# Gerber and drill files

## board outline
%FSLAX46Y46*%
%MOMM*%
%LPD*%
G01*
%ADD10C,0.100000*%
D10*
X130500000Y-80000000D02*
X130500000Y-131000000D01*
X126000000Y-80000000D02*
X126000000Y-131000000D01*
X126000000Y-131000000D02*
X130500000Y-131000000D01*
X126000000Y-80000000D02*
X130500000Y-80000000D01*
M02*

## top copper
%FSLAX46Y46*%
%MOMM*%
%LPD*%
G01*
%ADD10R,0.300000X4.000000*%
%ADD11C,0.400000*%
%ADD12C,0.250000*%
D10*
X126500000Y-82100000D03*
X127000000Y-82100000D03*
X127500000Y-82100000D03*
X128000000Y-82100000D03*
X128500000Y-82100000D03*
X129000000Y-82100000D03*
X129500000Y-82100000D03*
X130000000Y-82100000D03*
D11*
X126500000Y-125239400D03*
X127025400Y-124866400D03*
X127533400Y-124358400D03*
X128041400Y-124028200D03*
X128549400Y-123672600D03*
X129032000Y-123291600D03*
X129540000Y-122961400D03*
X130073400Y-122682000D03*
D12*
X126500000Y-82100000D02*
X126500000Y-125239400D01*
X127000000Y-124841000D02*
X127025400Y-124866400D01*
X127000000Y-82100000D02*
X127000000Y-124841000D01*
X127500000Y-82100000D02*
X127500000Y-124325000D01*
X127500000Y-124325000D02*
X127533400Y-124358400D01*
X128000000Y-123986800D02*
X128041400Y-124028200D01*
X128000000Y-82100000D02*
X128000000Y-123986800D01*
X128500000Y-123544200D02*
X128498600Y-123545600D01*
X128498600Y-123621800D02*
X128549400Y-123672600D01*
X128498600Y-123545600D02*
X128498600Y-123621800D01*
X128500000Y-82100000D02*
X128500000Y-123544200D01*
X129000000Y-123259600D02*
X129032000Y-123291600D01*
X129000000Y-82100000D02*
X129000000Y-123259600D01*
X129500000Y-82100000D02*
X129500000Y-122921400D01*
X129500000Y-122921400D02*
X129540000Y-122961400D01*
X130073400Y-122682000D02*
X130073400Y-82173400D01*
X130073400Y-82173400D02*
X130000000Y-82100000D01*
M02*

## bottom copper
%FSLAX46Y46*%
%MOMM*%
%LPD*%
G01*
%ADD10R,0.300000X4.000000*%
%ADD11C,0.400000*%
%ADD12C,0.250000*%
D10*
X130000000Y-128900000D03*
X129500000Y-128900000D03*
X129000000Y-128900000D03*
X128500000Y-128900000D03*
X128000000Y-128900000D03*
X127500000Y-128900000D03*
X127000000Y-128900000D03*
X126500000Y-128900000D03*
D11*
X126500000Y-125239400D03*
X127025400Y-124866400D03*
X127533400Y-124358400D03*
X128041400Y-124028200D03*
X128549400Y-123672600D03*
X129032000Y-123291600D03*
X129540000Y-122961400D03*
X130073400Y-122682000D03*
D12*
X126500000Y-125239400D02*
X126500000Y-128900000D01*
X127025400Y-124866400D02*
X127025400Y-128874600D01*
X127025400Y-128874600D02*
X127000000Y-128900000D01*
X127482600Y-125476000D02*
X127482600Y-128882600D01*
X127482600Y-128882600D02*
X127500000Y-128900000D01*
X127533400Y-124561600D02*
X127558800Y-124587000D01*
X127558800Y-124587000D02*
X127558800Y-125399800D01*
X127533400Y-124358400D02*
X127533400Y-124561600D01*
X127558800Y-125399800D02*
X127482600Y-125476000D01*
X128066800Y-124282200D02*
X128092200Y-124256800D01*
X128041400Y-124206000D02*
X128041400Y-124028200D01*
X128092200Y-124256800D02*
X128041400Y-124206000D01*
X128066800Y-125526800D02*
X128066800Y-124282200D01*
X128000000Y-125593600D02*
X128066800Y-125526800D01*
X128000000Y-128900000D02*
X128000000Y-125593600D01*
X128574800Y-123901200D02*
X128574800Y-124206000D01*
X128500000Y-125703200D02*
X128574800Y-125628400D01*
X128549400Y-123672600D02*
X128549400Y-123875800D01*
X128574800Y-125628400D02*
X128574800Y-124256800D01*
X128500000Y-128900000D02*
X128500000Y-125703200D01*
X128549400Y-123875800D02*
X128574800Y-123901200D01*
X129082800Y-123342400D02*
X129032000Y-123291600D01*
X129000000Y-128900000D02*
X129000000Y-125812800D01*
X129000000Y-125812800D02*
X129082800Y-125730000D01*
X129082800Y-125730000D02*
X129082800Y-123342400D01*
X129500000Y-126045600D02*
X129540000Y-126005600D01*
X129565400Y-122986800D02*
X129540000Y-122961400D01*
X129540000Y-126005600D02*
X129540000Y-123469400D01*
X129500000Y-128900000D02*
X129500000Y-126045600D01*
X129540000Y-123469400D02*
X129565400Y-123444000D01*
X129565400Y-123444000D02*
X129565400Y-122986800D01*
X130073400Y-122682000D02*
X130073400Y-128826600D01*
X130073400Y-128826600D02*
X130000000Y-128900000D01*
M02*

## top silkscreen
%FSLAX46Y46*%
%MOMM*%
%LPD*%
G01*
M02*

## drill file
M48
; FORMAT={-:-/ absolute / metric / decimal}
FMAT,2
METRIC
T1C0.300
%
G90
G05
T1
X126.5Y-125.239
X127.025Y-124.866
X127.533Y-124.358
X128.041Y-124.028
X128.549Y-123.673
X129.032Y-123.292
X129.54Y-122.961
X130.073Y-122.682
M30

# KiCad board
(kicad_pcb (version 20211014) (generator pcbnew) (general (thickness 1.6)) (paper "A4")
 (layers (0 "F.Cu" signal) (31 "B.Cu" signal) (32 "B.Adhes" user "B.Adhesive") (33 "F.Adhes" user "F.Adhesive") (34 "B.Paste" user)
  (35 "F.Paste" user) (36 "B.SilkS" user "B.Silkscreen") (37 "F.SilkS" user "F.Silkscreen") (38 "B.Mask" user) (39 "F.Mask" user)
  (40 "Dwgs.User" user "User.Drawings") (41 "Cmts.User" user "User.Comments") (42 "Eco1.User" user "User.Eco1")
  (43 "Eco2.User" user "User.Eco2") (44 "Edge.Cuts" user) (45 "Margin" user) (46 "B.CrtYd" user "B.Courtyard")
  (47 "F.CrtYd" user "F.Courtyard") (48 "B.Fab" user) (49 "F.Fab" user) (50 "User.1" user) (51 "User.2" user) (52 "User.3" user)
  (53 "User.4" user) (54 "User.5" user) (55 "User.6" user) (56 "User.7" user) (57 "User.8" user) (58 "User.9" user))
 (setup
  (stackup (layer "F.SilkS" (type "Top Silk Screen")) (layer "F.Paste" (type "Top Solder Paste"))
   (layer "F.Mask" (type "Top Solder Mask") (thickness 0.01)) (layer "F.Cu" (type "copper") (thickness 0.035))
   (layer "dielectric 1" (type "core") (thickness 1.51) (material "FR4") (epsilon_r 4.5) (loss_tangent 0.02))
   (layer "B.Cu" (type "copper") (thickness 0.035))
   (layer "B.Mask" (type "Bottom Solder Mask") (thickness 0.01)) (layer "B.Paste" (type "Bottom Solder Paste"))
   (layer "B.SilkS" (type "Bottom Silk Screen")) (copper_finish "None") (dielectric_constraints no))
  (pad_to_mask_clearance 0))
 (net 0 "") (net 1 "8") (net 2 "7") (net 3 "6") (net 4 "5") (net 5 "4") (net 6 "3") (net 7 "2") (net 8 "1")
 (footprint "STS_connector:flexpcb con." (layer "F.Cu") (at 126 84.1)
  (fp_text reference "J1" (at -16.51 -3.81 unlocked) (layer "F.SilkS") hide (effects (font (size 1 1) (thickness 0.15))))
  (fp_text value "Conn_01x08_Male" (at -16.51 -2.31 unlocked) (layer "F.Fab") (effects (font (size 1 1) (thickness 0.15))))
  (pad "1" smd rect (at 0.5 -2) (size 0.3 4) (layers "F.Cu" "F.Paste" "F.Mask") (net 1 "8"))
  (pad "2" smd rect (at 1 -2) (size 0.3 4) (layers "F.Cu" "F.Paste" "F.Mask") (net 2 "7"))
  (pad "3" smd rect (at 1.5 -2) (size 0.3 4) (layers "F.Cu" "F.Paste" "F.Mask") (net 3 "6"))
  (pad "4" smd rect (at 2 -2) (size 0.3 4) (layers "F.Cu" "F.Paste" "F.Mask") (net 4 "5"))
  (pad "5" smd rect (at 2.5 -2) (size 0.3 4) (layers "F.Cu" "F.Paste" "F.Mask") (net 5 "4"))
  (pad "6" smd rect (at 3 -2) (size 0.3 4) (layers "F.Cu" "F.Paste" "F.Mask") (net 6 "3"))
  (pad "7" smd rect (at 3.5 -2) (size 0.3 4) (layers "F.Cu" "F.Paste" "F.Mask") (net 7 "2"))
  (pad "8" smd rect (at 4 -2) (size 0.3 4) (layers "F.Cu" "F.Paste" "F.Mask") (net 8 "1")))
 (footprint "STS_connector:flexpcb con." (layer "B.Cu") (at 130.5 130.9 180)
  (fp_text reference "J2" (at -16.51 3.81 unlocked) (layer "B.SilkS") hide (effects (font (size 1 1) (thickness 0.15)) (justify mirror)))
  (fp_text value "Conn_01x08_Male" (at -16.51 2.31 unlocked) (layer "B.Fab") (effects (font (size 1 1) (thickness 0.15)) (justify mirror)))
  (pad "1" smd rect (at 0.5 2 180) (size 0.3 4) (layers "B.Cu" "B.Paste" "B.Mask") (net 8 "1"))
  (pad "2" smd rect (at 1 2 180) (size 0.3 4) (layers "B.Cu" "B.Paste" "B.Mask") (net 7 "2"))
  (pad "3" smd rect (at 1.5 2 180) (size 0.3 4) (layers "B.Cu" "B.Paste" "B.Mask") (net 6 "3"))
  (pad "4" smd rect (at 2 2 180) (size 0.3 4) (layers "B.Cu" "B.Paste" "B.Mask") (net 5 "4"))
  (pad "5" smd rect (at 2.5 2 180) (size 0.3 4) (layers "B.Cu" "B.Paste" "B.Mask") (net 4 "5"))
  (pad "6" smd rect (at 3 2 180) (size 0.3 4) (layers "B.Cu" "B.Paste" "B.Mask") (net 3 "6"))
  (pad "7" smd rect (at 3.5 2 180) (size 0.3 4) (layers "B.Cu" "B.Paste" "B.Mask") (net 2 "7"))
  (pad "8" smd rect (at 4 2 180) (size 0.3 4) (layers "B.Cu" "B.Paste" "B.Mask") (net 1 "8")))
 (gr_line (start 130.5 80) (end 130.5 131) (layer "Edge.Cuts") (width 0.1))
 (gr_line (start 126 80) (end 126 131) (layer "Edge.Cuts") (width 0.1))
 (gr_line (start 126 131) (end 130.5 131) (layer "Edge.Cuts") (width 0.1))
 (gr_line (start 126 80) (end 130.5 80) (layer "Edge.Cuts") (width 0.1))
 (segment (start 126.5 82.1) (end 126.5 125.2394) (width 0.25) (layer "F.Cu") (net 1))
 (via (at 126.5 125.2394) (size 0.4) (drill 0.3) (layers "F.Cu" "B.Cu") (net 1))
 (segment (start 126.5 125.2394) (end 126.5 128.9) (width 0.25) (layer "B.Cu") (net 1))
 (segment (start 127 124.841) (end 127.0254 124.8664) (width 0.25) (layer "F.Cu") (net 2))
 (segment (start 127 82.1) (end 127 124.841) (width 0.25) (layer "F.Cu") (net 2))
 (via (at 127.0254 124.8664) (size 0.4) (drill 0.3) (layers "F.Cu" "B.Cu") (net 2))
 (segment (start 127.0254 124.8664) (end 127.0254 128.8746) (width 0.25) (layer "B.Cu") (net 2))
 (segment (start 127.0254 128.8746) (end 127 128.9) (width 0.25) (layer "B.Cu") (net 2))
 (segment (start 127.5 82.1) (end 127.5 124.325) (width 0.25) (layer "F.Cu") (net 3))
 (segment (start 127.5 124.325) (end 127.5334 124.3584) (width 0.25) (layer "F.Cu") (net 3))
 (via (at 127.5334 124.3584) (size 0.4) (drill 0.3) (layers "F.Cu" "B.Cu") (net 3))
 (segment (start 127.4826 125.476) (end 127.4826 128.8826) (width 0.25) (layer "B.Cu") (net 3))
 (segment (start 127.4826 128.8826) (end 127.5 128.9) (width 0.25) (layer "B.Cu") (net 3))
 (segment (start 127.5334 124.5616) (end 127.5588 124.587) (width 0.25) (layer "B.Cu") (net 3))
 (segment (start 127.5588 124.587) (end 127.5588 125.3998) (width 0.25) (layer "B.Cu") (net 3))
 (segment (start 127.5334 124.3584) (end 127.5334 124.5616) (width 0.25) (layer "B.Cu") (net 3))
 (segment (start 127.5588 125.3998) (end 127.4826 125.476) (width 0.25) (layer "B.Cu") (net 3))
 (segment (start 128 123.9868) (end 128.0414 124.0282) (width 0.25) (layer "F.Cu") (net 4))
 (segment (start 128 82.1) (end 128 123.9868) (width 0.25) (layer "F.Cu") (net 4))
 (via (at 128.0414 124.0282) (size 0.4) (drill 0.3) (layers "F.Cu" "B.Cu") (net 4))
 (segment (start 128.0668 124.2822) (end 128.0922 124.2568) (width 0.25) (layer "B.Cu") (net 4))
 (segment (start 128.0414 124.206) (end 128.0414 124.0282) (width 0.25) (layer "B.Cu") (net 4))
 (segment (start 128.0922 124.2568) (end 128.0414 124.206) (width 0.25) (layer "B.Cu") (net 4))
 (segment (start 128.0668 125.5268) (end 128.0668 124.2822) (width 0.25) (layer "B.Cu") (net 4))
 (segment (start 128 125.5936) (end 128.0668 125.5268) (width 0.25) (layer "B.Cu") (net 4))
 (segment (start 128 128.9) (end 128 125.5936) (width 0.25) (layer "B.Cu") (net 4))
 (segment (start 128.5 123.5442) (end 128.4986 123.5456) (width 0.25) (layer "F.Cu") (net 5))
 (segment (start 128.4986 123.6218) (end 128.5494 123.6726) (width 0.25) (layer "F.Cu") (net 5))
 (segment (start 128.4986 123.5456) (end 128.4986 123.6218) (width 0.25) (layer "F.Cu") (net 5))
 (segment (start 128.5 82.1) (end 128.5 123.5442) (width 0.25) (layer "F.Cu") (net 5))
 (via (at 128.5494 123.6726) (size 0.4) (drill 0.3) (layers "F.Cu" "B.Cu") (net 5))
 (segment (start 128.5748 123.9012) (end 128.5748 124.206) (width 0.25) (layer "B.Cu") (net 5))
 (segment (start 128.5 125.7032) (end 128.5748 125.6284) (width 0.25) (layer "B.Cu") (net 5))
 (segment (start 128.5494 123.6726) (end 128.5494 123.8758) (width 0.25) (layer "B.Cu") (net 5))
 (segment (start 128.5748 125.6284) (end 128.5748 124.2568) (width 0.25) (layer "B.Cu") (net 5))
 (segment (start 128.5 128.9) (end 128.5 125.7032) (width 0.25) (layer "B.Cu") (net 5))
 (segment (start 128.5494 123.8758) (end 128.5748 123.9012) (width 0.25) (layer "B.Cu") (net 5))
 (segment (start 129 123.2596) (end 129.032 123.2916) (width 0.25) (layer "F.Cu") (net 6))
 (segment (start 129 82.1) (end 129 123.2596) (width 0.25) (layer "F.Cu") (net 6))
 (via (at 129.032 123.2916) (size 0.4) (drill 0.3) (layers "F.Cu" "B.Cu") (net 6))
 (segment (start 129.0828 123.3424) (end 129.032 123.2916) (width 0.25) (layer "B.Cu") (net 6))
 (segment (start 129 128.9) (end 129 125.8128) (width 0.25) (layer "B.Cu") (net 6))
 (segment (start 129 125.8128) (end 129.0828 125.73) (width 0.25) (layer "B.Cu") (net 6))
 (segment (start 129.0828 125.73) (end 129.0828 123.3424) (width 0.25) (layer "B.Cu") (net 6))
 (segment (start 129.5 82.1) (end 129.5 122.9214) (width 0.25) (layer "F.Cu") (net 7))
 (segment (start 129.5 122.9214) (end 129.54 122.9614) (width 0.25) (layer "F.Cu") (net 7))
 (via (at 129.54 122.9614) (size 0.4) (drill 0.3) (layers "F.Cu" "B.Cu") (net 7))
 (segment (start 129.5 126.0456) (end 129.54 126.0056) (width 0.25) (layer "B.Cu") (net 7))
 (segment (start 129.5654 122.9868) (end 129.54 122.9614) (width 0.25) (layer "B.Cu") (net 7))
 (segment (start 129.54 126.0056) (end 129.54 123.4694) (width 0.25) (layer "B.Cu") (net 7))
 (segment (start 129.5 128.9) (end 129.5 126.0456) (width 0.25) (layer "B.Cu") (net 7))
 (segment (start 129.54 123.4694) (end 129.5654 123.444) (width 0.25) (layer "B.Cu") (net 7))
 (segment (start 129.5654 123.444) (end 129.5654 122.9868) (width 0.25) (layer "B.Cu") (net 7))
 (segment (start 130.0734 122.682) (end 130.0734 82.1734) (width 0.25) (layer "F.Cu") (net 8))
 (segment (start 130.0734 82.1734) (end 130 82.1) (width 0.25) (layer "F.Cu") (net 8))
 (via (at 130.0734 122.682) (size 0.4) (drill 0.3) (layers "F.Cu" "B.Cu") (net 8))
 (segment (start 130.0734 122.682) (end 130.0734 128.8266) (width 0.25) (layer "B.Cu") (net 8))
 (segment (start 130.0734 128.8266) (end 130 128.9) (width 0.25) (layer "B.Cu") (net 8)))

